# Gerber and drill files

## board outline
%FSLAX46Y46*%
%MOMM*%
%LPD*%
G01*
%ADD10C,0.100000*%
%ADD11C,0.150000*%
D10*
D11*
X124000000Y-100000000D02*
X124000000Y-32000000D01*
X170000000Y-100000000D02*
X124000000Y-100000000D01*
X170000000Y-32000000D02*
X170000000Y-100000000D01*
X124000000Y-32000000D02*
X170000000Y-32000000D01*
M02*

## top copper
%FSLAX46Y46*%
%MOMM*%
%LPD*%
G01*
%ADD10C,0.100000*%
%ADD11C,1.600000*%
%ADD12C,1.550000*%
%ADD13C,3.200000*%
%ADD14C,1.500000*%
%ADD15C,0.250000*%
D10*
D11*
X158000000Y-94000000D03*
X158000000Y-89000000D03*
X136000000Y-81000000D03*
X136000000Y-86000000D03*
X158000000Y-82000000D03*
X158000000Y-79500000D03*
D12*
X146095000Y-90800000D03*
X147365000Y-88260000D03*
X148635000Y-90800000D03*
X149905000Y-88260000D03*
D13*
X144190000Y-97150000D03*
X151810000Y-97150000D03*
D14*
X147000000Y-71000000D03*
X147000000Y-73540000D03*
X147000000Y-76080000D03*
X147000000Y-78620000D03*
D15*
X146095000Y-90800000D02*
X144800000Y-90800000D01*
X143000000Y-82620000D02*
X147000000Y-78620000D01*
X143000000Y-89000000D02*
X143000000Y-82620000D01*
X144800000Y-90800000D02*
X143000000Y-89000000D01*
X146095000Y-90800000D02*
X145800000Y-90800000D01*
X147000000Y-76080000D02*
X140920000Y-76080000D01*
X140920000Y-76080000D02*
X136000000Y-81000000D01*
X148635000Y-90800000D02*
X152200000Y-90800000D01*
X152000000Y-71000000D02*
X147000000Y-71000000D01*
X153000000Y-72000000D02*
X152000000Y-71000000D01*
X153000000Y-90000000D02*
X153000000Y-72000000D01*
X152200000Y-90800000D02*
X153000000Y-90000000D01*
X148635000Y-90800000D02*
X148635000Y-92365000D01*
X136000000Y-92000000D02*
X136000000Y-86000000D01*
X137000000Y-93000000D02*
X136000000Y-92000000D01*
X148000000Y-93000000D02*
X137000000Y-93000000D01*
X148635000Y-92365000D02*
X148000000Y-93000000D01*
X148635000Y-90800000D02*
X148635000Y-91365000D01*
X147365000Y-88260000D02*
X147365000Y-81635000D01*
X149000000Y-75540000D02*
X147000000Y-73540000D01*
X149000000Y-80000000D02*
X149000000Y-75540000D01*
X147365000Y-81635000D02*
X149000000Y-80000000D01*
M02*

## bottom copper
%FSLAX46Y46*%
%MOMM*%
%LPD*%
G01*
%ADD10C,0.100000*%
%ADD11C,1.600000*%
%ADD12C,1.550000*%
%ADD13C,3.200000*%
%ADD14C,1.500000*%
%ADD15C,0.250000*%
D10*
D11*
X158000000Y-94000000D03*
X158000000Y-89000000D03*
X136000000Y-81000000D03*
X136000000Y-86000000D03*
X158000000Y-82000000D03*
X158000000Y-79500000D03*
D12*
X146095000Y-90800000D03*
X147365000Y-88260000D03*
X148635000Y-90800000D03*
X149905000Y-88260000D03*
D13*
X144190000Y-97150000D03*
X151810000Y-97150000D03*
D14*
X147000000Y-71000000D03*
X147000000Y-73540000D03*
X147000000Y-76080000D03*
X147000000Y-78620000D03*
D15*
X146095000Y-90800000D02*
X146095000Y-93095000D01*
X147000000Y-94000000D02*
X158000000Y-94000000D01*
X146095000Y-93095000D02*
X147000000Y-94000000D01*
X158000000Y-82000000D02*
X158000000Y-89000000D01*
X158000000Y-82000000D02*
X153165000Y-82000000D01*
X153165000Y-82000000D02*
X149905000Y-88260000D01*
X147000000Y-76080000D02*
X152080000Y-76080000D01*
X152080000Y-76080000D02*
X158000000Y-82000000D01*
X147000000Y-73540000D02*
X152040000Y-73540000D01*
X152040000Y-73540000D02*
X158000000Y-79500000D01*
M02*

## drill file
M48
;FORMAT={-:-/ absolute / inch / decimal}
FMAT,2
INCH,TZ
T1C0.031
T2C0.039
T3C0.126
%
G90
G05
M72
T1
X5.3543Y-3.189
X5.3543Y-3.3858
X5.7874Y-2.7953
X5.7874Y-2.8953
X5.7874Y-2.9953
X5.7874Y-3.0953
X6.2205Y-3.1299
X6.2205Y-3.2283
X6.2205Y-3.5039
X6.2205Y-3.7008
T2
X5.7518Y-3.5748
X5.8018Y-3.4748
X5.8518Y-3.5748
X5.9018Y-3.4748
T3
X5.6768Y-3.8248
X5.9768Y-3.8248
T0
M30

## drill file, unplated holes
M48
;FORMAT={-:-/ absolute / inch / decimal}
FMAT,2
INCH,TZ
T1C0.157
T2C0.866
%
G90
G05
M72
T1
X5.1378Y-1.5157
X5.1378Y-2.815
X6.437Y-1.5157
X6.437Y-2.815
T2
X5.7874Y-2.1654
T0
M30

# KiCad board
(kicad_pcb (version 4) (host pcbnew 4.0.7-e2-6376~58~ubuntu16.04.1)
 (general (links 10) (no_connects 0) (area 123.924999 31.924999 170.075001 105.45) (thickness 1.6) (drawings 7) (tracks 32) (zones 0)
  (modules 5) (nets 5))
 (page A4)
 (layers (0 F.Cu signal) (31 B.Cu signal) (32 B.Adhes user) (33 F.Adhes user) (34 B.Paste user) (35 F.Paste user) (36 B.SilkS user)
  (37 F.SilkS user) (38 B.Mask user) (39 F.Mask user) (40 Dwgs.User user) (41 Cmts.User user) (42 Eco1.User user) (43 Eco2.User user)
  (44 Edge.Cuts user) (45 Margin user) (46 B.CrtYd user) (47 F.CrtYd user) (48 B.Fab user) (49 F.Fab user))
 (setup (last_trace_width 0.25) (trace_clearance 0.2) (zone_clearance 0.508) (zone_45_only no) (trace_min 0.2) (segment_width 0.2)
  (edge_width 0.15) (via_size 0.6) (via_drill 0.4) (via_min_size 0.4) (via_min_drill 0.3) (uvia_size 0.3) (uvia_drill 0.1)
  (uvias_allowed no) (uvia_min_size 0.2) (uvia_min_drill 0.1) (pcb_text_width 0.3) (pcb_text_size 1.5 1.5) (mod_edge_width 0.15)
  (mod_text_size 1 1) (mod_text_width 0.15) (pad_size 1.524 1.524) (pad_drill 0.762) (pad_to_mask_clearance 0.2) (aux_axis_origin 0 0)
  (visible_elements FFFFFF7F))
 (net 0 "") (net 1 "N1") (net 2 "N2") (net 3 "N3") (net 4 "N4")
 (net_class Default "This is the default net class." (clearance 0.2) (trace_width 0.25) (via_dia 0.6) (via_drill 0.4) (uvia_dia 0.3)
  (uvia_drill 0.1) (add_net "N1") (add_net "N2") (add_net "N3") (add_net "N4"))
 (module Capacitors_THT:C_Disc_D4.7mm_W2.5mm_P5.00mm (layer F.Cu) (at 158 94 90)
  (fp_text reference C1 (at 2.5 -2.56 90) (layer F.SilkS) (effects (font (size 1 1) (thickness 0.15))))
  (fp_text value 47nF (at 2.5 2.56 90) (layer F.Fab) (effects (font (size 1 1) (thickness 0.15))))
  (pad 1 thru_hole circle (at 0 0 90) (size 1.6 1.6) (drill 0.8) (layers *.Cu *.Mask) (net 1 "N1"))
  (pad 2 thru_hole circle (at 5 0 90) (size 1.6 1.6) (drill 0.8) (layers *.Cu *.Mask) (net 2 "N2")))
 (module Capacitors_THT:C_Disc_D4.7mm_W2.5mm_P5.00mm (layer F.Cu) (at 136 81 270)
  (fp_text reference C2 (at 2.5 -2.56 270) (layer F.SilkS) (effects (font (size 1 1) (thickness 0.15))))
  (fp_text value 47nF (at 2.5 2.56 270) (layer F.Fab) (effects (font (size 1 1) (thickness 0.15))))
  (pad 1 thru_hole circle (at 0 0 270) (size 1.6 1.6) (drill 0.8) (layers *.Cu *.Mask) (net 2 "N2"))
  (pad 2 thru_hole circle (at 5 0 270) (size 1.6 1.6) (drill 0.8) (layers *.Cu *.Mask) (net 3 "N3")))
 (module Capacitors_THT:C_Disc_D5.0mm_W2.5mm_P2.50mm (layer F.Cu) (at 158 82 90)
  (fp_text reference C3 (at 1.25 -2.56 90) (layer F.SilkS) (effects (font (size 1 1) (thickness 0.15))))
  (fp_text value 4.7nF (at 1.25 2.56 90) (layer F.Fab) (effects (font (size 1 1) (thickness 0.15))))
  (pad 1 thru_hole circle (at 0 0 90) (size 1.6 1.6) (drill 0.8) (layers *.Cu *.Mask) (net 2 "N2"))
  (pad 2 thru_hole circle (at 2.5 0 90) (size 1.6 1.6) (drill 0.8) (layers *.Cu *.Mask) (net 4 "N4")))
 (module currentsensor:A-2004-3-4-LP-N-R (layer F.Cu) (at 148 105)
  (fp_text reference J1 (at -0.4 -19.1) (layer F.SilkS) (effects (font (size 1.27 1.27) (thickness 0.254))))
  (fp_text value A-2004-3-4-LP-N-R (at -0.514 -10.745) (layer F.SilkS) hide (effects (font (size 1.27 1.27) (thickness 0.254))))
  (pad 1 thru_hole circle (at -1.905 -14.2 90) (size 1.55 1.55) (drill 1) (layers *.Cu *.Mask F.SilkS) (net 1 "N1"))
  (pad 2 thru_hole circle (at -0.635 -16.74 90) (size 1.55 1.55) (drill 1) (layers *.Cu *.Mask F.SilkS) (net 4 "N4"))
  (pad 3 thru_hole circle (at 0.635 -14.2 90) (size 1.55 1.55) (drill 1) (layers *.Cu *.Mask F.SilkS) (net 3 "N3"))
  (pad 4 thru_hole circle (at 1.905 -16.74 90) (size 1.55 1.55) (drill 1) (layers *.Cu *.Mask F.SilkS) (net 2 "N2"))
  (pad 5 thru_hole circle (at -3.81 -7.85 90) (size 3.2 3.2) (drill 3.2) (layers *.Cu *.Mask F.SilkS))
  (pad 6 thru_hole circle (at 3.81 -7.85 90) (size 3.2 3.2) (drill 3.2) (layers *.Cu *.Mask F.SilkS)))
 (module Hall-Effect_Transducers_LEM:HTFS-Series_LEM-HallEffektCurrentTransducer (layer F.Cu) (at 147 55)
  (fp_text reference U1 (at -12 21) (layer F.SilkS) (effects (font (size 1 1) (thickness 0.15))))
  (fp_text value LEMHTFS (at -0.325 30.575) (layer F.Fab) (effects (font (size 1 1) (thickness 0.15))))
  (pad "" np_thru_hole circle (at 0 0) (size 22 22) (drill 22) (layers *.Cu *.Mask))
  (pad "" np_thru_hole circle (at 16.5 -16.5) (size 4 4) (drill 4) (layers *.Cu *.Mask))
  (pad "" np_thru_hole circle (at -16.5 -16.5) (size 4 4) (drill 4) (layers *.Cu *.Mask))
  (pad "" np_thru_hole circle (at -16.5 16.5) (size 4 4) (drill 4) (layers *.Cu *.Mask))
  (pad "" np_thru_hole circle (at 16.5 16.5) (size 4 4) (drill 4) (layers *.Cu *.Mask))
  (pad 4 thru_hole circle (at 0 16) (size 1.5 1.5) (drill 0.8) (layers *.Cu *.Mask) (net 3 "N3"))
  (pad 3 thru_hole circle (at 0 18.54) (size 1.5 1.5) (drill 0.8) (layers *.Cu *.Mask) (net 4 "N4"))
  (pad 2 thru_hole circle (at 0 21.08) (size 1.5 1.5) (drill 0.8) (layers *.Cu *.Mask) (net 2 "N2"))
  (pad 1 thru_hole circle (at 0 23.62) (size 1.5 1.5) (drill 0.8) (layers *.Cu *.Mask) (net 1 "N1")))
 (gr_line (start 124 100) (end 124 32) (angle 90) (layer Edge.Cuts) (width 0.15))
 (gr_line (start 170 100) (end 124 100) (angle 90) (layer Edge.Cuts) (width 0.15))
 (gr_line (start 170 32) (end 170 100) (angle 90) (layer Edge.Cuts) (width 0.15))
 (gr_line (start 124 32) (end 170 32) (angle 90) (layer Edge.Cuts) (width 0.15))
 (segment (start 146.095 90.8) (end 144.8 90.8) (width 0.25) (layer F.Cu) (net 1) (status 400000))
 (segment (start 143 82.62) (end 147 78.62) (width 0.25) (layer F.Cu) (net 1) (status 800000))
 (segment (start 143 89) (end 143 82.62) (width 0.25) (layer F.Cu) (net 1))
 (segment (start 144.8 90.8) (end 143 89) (width 0.25) (layer F.Cu) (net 1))
 (segment (start 146.095 90.8) (end 146.095 93.095) (width 0.25) (layer B.Cu) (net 1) (status 400000))
 (segment (start 147 94) (end 158 94) (width 0.25) (layer B.Cu) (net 1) (status 800000))
 (segment (start 146.095 93.095) (end 147 94) (width 0.25) (layer B.Cu) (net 1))
 (segment (start 146.095 90.8) (end 145.8 90.8) (width 0.25) (layer F.Cu) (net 1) (status 30))
 (segment (start 158 82) (end 158 89) (width 0.25) (layer B.Cu) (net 2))
 (segment (start 158 82) (end 153.165 82) (width 0.25) (layer B.Cu) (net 2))
 (segment (start 153.165 82) (end 149.905 88.26) (width 0.25) (layer B.Cu) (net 2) (status 20))
 (segment (start 147 76.08) (end 152.08 76.08) (width 0.25) (layer B.Cu) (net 2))
 (segment (start 152.08 76.08) (end 158 82) (width 0.25) (layer B.Cu) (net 2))
 (segment (start 147 76.08) (end 140.92 76.08) (width 0.25) (layer F.Cu) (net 2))
 (segment (start 140.92 76.08) (end 136 81) (width 0.25) (layer F.Cu) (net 2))
 (segment (start 148.635 90.8) (end 152.2 90.8) (width 0.25) (layer F.Cu) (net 3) (status 400000))
 (segment (start 152 71) (end 147 71) (width 0.25) (layer F.Cu) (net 3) (status 800000))
 (segment (start 153 72) (end 152 71) (width 0.25) (layer F.Cu) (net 3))
 (segment (start 153 90) (end 153 72) (width 0.25) (layer F.Cu) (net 3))
 (segment (start 152.2 90.8) (end 153 90) (width 0.25) (layer F.Cu) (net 3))
 (segment (start 148.635 90.8) (end 148.635 92.365) (width 0.25) (layer F.Cu) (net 3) (status 400000))
 (segment (start 136 92) (end 136 86) (width 0.25) (layer F.Cu) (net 3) (status 800000))
 (segment (start 137 93) (end 136 92) (width 0.25) (layer F.Cu) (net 3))
 (segment (start 148 93) (end 137 93) (width 0.25) (layer F.Cu) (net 3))
 (segment (start 148.635 92.365) (end 148 93) (width 0.25) (layer F.Cu) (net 3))
 (segment (start 148.635 90.8) (end 148.635 91.365) (width 0.25) (layer F.Cu) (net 3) (status 30))
 (segment (start 147.365 88.26) (end 147.365 81.635) (width 0.25) (layer F.Cu) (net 4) (status 10))
 (segment (start 149 75.54) (end 147 73.54) (width 0.25) (layer F.Cu) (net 4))
 (segment (start 149 80) (end 149 75.54) (width 0.25) (layer F.Cu) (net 4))
 (segment (start 147.365 81.635) (end 149 80) (width 0.25) (layer F.Cu) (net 4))
 (segment (start 147 73.54) (end 152.04 73.54) (width 0.25) (layer B.Cu) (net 4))
 (segment (start 152.04 73.54) (end 158 79.5) (width 0.25) (layer B.Cu) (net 4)))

